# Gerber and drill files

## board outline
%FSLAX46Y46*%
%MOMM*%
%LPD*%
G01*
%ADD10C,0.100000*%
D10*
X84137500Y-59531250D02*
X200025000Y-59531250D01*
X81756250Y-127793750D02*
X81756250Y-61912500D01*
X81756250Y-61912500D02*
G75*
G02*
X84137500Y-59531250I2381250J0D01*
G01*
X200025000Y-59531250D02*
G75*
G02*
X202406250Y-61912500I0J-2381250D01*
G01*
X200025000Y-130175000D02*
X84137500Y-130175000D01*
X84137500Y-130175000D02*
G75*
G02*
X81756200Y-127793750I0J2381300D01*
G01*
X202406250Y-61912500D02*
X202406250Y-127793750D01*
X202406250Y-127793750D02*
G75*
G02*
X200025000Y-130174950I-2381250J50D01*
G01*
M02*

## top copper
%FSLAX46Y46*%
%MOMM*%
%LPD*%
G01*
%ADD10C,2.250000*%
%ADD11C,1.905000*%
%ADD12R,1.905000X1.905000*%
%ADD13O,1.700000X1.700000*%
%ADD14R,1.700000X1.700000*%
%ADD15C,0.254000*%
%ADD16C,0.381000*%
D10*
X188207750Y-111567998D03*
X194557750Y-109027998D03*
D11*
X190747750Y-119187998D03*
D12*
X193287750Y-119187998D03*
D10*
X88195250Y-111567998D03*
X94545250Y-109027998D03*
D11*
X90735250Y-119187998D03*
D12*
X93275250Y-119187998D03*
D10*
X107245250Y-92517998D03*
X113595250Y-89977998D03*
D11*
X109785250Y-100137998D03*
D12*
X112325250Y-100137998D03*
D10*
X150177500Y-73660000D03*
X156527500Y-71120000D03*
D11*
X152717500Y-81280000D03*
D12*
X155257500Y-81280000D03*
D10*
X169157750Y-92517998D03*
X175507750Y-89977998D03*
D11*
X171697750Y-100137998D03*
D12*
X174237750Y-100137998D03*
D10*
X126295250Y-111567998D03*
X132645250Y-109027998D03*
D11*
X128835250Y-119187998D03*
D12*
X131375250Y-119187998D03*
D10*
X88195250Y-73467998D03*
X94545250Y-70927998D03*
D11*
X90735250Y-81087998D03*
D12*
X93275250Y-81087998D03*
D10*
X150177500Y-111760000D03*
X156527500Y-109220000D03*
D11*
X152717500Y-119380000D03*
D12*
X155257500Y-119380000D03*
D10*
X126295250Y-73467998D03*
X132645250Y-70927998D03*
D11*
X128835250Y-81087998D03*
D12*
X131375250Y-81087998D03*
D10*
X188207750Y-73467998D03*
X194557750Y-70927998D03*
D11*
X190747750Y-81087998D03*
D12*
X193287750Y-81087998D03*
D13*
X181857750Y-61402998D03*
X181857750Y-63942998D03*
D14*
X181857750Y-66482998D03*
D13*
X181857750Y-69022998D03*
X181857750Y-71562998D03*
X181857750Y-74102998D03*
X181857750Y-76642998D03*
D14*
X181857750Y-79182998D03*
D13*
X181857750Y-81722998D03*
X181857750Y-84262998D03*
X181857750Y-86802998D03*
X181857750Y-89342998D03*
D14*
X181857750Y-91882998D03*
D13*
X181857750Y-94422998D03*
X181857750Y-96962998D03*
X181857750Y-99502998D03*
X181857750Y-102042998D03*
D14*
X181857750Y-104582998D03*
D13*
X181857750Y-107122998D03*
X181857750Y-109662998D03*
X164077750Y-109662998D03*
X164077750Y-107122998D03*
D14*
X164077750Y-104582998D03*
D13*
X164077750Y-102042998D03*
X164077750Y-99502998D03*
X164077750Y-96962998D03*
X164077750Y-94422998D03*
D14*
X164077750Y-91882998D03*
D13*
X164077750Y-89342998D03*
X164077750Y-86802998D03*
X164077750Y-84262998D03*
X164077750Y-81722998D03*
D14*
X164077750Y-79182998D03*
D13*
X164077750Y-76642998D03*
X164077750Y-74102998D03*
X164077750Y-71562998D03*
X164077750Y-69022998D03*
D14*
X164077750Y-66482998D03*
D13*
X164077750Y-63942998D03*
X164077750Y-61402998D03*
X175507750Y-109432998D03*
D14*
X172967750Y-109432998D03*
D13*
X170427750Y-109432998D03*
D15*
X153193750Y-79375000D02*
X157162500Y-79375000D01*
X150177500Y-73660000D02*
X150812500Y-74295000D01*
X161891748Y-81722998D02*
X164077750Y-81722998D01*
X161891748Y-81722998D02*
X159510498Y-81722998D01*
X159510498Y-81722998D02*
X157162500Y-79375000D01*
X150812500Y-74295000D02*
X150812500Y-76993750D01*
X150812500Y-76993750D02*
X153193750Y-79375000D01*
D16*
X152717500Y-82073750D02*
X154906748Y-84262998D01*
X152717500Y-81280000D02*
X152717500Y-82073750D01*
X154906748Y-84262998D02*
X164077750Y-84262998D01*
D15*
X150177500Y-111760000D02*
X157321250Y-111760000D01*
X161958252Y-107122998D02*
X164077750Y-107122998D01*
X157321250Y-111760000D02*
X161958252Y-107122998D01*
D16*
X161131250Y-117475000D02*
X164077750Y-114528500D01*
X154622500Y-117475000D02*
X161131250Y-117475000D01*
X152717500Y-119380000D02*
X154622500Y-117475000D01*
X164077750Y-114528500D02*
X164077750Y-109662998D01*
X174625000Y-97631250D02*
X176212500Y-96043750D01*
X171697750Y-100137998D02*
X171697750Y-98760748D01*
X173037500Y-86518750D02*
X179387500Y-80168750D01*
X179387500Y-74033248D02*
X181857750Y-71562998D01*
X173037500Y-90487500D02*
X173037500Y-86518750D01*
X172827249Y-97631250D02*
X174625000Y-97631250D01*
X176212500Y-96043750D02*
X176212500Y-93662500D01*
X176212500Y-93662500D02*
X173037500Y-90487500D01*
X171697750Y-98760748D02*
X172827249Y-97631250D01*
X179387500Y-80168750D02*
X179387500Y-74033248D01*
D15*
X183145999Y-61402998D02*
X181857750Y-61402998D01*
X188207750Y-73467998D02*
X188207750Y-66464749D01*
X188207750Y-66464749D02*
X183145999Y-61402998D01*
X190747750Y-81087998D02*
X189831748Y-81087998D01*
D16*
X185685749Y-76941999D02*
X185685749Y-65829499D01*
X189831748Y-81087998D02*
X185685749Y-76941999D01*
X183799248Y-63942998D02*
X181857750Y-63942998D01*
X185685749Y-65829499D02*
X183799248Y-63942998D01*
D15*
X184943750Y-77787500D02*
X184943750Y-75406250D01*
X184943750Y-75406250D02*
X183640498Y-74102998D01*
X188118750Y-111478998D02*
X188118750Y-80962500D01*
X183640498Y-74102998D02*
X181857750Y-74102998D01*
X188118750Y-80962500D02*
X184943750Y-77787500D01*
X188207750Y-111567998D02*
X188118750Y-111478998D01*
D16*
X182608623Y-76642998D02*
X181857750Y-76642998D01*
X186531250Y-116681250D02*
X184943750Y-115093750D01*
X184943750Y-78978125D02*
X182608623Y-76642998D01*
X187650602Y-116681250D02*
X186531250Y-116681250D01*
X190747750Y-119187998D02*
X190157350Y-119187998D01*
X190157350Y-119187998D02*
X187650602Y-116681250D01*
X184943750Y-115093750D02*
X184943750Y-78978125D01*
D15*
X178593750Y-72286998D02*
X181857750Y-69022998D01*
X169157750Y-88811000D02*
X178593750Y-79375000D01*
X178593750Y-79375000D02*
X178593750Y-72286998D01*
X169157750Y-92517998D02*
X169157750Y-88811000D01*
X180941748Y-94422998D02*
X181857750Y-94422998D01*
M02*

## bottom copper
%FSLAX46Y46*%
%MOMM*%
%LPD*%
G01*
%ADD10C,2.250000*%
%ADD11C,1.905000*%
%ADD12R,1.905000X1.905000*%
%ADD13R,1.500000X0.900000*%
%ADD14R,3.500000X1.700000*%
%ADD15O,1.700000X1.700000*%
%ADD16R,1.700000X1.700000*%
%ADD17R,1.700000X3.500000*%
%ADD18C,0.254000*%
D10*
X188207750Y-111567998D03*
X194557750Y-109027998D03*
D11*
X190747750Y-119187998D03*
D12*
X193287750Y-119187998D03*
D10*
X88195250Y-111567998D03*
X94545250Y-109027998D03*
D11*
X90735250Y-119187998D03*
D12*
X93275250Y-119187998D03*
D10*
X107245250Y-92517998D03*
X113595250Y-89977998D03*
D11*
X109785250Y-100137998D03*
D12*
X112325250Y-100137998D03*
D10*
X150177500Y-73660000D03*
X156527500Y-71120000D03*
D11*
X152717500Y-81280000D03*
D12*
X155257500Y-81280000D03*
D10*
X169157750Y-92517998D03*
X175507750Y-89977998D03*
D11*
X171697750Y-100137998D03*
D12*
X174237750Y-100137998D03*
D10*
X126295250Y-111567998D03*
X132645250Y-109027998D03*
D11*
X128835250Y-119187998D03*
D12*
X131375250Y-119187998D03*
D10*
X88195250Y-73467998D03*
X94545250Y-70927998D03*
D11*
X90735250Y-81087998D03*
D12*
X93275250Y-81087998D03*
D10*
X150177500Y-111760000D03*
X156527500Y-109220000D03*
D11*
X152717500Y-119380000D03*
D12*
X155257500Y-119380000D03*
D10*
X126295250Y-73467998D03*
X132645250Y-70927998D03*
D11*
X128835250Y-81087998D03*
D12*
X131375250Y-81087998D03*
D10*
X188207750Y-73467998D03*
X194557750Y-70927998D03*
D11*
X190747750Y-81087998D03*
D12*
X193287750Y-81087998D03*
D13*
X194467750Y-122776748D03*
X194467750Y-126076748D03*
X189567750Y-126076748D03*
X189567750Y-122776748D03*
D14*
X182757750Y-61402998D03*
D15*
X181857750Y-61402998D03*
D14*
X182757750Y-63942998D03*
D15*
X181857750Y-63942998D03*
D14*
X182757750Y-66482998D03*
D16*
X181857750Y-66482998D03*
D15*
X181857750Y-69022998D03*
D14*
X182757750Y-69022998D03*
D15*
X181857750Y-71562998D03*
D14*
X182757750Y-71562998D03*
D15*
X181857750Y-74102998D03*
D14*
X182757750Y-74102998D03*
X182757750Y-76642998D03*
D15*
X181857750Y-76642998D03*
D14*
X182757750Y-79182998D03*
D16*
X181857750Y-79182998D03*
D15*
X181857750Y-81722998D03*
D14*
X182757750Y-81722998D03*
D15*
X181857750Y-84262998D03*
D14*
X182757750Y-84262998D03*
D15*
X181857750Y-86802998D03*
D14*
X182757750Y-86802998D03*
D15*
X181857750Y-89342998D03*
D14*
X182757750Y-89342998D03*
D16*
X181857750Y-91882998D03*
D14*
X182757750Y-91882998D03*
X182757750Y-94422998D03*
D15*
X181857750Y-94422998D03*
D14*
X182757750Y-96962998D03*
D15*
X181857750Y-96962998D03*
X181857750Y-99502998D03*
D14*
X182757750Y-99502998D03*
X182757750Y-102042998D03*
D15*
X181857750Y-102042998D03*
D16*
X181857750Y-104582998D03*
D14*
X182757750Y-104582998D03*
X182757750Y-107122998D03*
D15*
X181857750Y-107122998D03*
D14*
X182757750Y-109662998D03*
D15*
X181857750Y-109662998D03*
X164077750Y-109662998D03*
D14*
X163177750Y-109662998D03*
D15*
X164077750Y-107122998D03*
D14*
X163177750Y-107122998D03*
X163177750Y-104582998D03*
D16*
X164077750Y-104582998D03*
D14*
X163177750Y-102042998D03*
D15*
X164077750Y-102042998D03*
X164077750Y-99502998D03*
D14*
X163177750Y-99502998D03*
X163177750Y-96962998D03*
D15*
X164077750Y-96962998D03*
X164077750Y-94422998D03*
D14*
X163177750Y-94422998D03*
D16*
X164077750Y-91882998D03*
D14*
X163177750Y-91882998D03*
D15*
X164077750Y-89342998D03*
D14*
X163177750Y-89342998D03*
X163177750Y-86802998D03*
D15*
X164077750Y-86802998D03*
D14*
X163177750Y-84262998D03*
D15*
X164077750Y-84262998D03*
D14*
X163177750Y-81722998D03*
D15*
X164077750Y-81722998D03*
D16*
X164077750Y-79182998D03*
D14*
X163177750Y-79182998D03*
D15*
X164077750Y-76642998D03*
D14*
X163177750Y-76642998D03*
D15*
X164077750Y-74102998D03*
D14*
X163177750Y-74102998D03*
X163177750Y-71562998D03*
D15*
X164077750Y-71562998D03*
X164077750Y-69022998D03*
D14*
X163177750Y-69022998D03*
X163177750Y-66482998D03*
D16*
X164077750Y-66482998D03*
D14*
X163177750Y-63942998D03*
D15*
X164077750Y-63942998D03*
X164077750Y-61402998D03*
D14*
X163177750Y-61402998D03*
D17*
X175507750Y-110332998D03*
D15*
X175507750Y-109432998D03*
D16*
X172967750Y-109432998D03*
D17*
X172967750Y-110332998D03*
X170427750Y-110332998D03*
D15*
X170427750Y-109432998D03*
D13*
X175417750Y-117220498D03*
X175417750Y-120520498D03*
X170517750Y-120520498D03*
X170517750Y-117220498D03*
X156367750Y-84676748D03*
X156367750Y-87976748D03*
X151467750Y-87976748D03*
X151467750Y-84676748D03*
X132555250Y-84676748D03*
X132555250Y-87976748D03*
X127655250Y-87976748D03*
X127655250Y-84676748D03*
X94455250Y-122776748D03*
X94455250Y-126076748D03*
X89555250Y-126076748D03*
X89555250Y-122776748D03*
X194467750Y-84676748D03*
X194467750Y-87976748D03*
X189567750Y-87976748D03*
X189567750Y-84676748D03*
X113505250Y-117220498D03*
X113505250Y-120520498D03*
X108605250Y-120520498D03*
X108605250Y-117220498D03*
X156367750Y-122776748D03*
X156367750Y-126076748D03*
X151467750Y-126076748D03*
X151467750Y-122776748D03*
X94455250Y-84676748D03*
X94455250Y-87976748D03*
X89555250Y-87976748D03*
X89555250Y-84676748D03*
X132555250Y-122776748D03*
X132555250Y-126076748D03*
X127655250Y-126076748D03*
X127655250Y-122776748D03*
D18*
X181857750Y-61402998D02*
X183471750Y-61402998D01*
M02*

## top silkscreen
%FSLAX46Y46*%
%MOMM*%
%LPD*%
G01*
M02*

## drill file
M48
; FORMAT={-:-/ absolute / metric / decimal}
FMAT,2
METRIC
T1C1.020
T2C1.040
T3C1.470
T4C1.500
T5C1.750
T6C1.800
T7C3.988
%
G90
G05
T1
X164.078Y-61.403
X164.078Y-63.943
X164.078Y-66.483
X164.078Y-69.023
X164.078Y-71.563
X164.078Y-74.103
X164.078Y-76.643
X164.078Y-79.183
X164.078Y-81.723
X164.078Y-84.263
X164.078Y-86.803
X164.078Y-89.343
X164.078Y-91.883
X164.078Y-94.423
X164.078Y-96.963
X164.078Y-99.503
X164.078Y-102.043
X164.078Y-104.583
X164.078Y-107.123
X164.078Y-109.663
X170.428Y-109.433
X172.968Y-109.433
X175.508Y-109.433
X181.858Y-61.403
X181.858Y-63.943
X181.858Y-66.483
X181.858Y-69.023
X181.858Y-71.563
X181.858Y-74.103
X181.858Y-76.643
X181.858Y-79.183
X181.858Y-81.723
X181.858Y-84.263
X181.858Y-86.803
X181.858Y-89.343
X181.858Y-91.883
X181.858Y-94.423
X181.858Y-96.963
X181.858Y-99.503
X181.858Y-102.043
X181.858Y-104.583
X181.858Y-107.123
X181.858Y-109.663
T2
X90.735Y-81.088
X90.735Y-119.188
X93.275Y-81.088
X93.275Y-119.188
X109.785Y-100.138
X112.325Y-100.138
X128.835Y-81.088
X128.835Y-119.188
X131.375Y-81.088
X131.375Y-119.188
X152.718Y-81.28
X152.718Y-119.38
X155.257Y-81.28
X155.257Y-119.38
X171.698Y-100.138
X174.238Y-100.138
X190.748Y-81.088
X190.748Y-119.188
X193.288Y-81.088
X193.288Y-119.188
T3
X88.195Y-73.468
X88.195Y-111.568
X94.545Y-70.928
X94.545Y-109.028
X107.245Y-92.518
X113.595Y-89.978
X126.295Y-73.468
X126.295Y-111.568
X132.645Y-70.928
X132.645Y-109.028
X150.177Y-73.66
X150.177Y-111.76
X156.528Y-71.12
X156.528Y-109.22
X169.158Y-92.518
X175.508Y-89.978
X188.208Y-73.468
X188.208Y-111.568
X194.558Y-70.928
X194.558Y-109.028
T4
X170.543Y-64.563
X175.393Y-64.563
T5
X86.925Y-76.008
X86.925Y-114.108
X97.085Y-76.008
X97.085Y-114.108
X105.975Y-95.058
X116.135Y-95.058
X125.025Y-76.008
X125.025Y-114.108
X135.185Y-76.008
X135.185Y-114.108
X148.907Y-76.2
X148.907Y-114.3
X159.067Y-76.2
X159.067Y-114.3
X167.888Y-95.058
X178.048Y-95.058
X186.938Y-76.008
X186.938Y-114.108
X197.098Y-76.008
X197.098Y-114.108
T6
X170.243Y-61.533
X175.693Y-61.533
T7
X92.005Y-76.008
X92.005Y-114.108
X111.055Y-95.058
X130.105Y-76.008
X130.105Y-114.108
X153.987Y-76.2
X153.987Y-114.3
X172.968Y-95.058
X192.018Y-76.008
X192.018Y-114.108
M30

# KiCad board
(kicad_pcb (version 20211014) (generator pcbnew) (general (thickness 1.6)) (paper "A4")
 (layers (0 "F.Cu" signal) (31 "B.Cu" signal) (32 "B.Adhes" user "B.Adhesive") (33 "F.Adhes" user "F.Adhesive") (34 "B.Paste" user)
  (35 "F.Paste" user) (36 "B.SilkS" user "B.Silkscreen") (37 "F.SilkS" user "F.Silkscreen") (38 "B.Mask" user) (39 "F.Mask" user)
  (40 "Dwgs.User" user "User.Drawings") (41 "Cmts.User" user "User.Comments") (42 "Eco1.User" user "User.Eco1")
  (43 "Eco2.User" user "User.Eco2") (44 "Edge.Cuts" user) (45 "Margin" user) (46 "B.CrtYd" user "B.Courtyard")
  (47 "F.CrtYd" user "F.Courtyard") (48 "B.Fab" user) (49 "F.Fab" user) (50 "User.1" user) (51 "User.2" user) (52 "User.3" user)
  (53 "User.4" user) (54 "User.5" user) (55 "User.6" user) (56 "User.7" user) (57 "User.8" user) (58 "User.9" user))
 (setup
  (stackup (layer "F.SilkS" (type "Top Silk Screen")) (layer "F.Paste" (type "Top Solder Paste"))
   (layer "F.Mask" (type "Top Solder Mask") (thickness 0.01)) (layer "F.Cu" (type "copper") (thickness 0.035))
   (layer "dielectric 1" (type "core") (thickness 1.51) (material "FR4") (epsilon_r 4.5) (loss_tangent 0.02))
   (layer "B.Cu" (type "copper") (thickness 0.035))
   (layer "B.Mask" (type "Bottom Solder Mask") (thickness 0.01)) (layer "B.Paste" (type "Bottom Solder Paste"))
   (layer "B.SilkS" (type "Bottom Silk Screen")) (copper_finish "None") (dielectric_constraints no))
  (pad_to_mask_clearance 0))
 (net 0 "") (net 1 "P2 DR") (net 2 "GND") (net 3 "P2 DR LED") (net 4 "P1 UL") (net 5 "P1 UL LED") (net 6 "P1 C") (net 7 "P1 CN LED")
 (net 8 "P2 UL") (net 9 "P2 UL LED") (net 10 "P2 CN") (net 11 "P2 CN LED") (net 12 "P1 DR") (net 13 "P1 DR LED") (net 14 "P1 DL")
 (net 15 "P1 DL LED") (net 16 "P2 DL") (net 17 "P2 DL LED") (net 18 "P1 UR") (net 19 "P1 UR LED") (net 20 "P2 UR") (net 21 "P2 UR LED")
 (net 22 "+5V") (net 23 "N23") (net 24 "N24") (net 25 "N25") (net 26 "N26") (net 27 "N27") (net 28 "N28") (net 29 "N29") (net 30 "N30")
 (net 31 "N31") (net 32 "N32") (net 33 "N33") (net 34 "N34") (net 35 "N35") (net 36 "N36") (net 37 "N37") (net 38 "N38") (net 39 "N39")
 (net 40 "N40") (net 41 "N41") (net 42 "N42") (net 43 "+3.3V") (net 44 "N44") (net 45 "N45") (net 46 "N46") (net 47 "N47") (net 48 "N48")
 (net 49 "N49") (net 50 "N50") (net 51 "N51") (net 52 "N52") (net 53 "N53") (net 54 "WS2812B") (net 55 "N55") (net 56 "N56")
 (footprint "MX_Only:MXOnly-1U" (layer "F.Cu") (at 192.01775 114.107998)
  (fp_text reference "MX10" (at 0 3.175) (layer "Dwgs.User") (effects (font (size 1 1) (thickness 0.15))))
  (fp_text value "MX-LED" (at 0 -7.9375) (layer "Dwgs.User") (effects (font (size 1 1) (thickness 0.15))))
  (pad "" np_thru_hole circle locked (at 0 0) (size 3.9878 3.9878) (drill 3.9878) (layers *.Cu *.Mask))
  (pad "" np_thru_hole circle locked (at 5.08 0 48.0996) (size 1.75 1.75) (drill 1.75) (layers *.Cu *.Mask))
  (pad "" np_thru_hole circle locked (at -5.08 0 48.0996) (size 1.75 1.75) (drill 1.75) (layers *.Cu *.Mask))
  (pad "1" thru_hole circle locked (at -3.81 -2.54) (size 2.25 2.25) (drill 1.47) (layers *.Cu "B.Mask") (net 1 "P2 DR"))
  (pad "2" thru_hole circle locked (at 2.54 -5.08) (size 2.25 2.25) (drill 1.47) (layers *.Cu "B.Mask") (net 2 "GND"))
  (pad "3" thru_hole circle locked (at -1.27 5.08) (size 1.905 1.905) (drill 1.04) (layers *.Cu "B.Mask") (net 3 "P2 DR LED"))
  (pad "4" thru_hole rect locked (at 1.27 5.08) (size 1.905 1.905) (drill 1.04) (layers *.Cu "B.Mask") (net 2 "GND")))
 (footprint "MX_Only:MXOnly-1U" (layer "F.Cu") (at 92.00525 114.107998)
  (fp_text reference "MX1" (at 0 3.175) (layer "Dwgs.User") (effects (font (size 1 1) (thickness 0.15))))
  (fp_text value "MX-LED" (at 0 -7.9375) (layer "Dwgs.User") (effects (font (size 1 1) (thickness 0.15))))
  (pad "" np_thru_hole circle locked (at -5.08 0 48.0996) (size 1.75 1.75) (drill 1.75) (layers *.Cu *.Mask))
  (pad "" np_thru_hole circle locked (at 5.08 0 48.0996) (size 1.75 1.75) (drill 1.75) (layers *.Cu *.Mask))
  (pad "" np_thru_hole circle locked (at 0 0) (size 3.9878 3.9878) (drill 3.9878) (layers *.Cu *.Mask))
  (pad "1" thru_hole circle locked (at -3.81 -2.54) (size 2.25 2.25) (drill 1.47) (layers *.Cu "B.Mask") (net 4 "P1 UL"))
  (pad "2" thru_hole circle locked (at 2.54 -5.08) (size 2.25 2.25) (drill 1.47) (layers *.Cu "B.Mask") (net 2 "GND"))
  (pad "3" thru_hole circle locked (at -1.27 5.08) (size 1.905 1.905) (drill 1.04) (layers *.Cu "B.Mask") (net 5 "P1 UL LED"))
  (pad "4" thru_hole rect locked (at 1.27 5.08) (size 1.905 1.905) (drill 1.04) (layers *.Cu "B.Mask") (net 2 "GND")))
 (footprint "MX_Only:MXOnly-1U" (layer "F.Cu") (at 111.05525 95.057998)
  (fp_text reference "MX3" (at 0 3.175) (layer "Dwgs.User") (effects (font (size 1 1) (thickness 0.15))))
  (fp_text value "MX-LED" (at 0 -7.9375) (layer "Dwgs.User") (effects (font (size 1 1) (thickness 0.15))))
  (pad "" np_thru_hole circle locked (at -5.08 0 48.0996) (size 1.75 1.75) (drill 1.75) (layers *.Cu *.Mask))
  (pad "" np_thru_hole circle locked (at 5.08 0 48.0996) (size 1.75 1.75) (drill 1.75) (layers *.Cu *.Mask))
  (pad "" np_thru_hole circle locked (at 0 0) (size 3.9878 3.9878) (drill 3.9878) (layers *.Cu *.Mask))
  (pad "1" thru_hole circle locked (at -3.81 -2.54) (size 2.25 2.25) (drill 1.47) (layers *.Cu "B.Mask") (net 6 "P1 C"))
  (pad "2" thru_hole circle locked (at 2.54 -5.08) (size 2.25 2.25) (drill 1.47) (layers *.Cu "B.Mask") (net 2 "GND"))
  (pad "3" thru_hole circle locked (at -1.27 5.08) (size 1.905 1.905) (drill 1.04) (layers *.Cu "B.Mask") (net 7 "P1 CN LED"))
  (pad "4" thru_hole rect locked (at 1.27 5.08) (size 1.905 1.905) (drill 1.04) (layers *.Cu "B.Mask") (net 2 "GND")))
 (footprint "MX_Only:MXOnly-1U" (layer "F.Cu") (at 153.9875 76.2)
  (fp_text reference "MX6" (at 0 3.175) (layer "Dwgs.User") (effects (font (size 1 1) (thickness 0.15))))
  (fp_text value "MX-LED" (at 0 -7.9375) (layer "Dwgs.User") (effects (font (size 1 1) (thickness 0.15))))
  (pad "" np_thru_hole circle locked (at -5.08 0 48.0996) (size 1.75 1.75) (drill 1.75) (layers *.Cu *.Mask))
  (pad "" np_thru_hole circle locked (at 0 0) (size 3.9878 3.9878) (drill 3.9878) (layers *.Cu *.Mask))
  (pad "" np_thru_hole circle locked (at 5.08 0 48.0996) (size 1.75 1.75) (drill 1.75) (layers *.Cu *.Mask))
  (pad "1" thru_hole circle locked (at -3.81 -2.54) (size 2.25 2.25) (drill 1.47) (layers *.Cu "B.Mask") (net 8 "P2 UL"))
  (pad "2" thru_hole circle locked (at 2.54 -5.08) (size 2.25 2.25) (drill 1.47) (layers *.Cu "B.Mask") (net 2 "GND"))
  (pad "3" thru_hole circle locked (at -1.27 5.08) (size 1.905 1.905) (drill 1.04) (layers *.Cu "B.Mask") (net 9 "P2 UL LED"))
  (pad "4" thru_hole rect locked (at 1.27 5.08) (size 1.905 1.905) (drill 1.04) (layers *.Cu "B.Mask") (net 2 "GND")))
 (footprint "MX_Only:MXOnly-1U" (layer "F.Cu") (at 172.96775 95.057998)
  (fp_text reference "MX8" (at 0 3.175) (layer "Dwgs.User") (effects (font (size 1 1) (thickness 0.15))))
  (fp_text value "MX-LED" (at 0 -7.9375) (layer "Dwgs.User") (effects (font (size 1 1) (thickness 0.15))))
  (pad "" np_thru_hole circle locked (at 5.08 0 48.0996) (size 1.75 1.75) (drill 1.75) (layers *.Cu *.Mask))
  (pad "" np_thru_hole circle locked (at -5.08 0 48.0996) (size 1.75 1.75) (drill 1.75) (layers *.Cu *.Mask))
  (pad "" np_thru_hole circle locked (at 0 0) (size 3.9878 3.9878) (drill 3.9878) (layers *.Cu *.Mask))
  (pad "1" thru_hole circle locked (at -3.81 -2.54) (size 2.25 2.25) (drill 1.47) (layers *.Cu "B.Mask") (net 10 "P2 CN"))
  (pad "2" thru_hole circle locked (at 2.54 -5.08) (size 2.25 2.25) (drill 1.47) (layers *.Cu "B.Mask") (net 2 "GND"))
  (pad "3" thru_hole circle locked (at -1.27 5.08) (size 1.905 1.905) (drill 1.04) (layers *.Cu "B.Mask") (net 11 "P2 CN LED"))
  (pad "4" thru_hole rect locked (at 1.27 5.08) (size 1.905 1.905) (drill 1.04) (layers *.Cu "B.Mask") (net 2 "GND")))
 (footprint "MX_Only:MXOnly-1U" (layer "F.Cu") (at 130.10525 114.107998)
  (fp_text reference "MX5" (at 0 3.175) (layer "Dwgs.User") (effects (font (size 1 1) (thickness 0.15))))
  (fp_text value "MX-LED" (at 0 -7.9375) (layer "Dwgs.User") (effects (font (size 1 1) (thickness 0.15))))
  (pad "" np_thru_hole circle locked (at 5.08 0 48.0996) (size 1.75 1.75) (drill 1.75) (layers *.Cu *.Mask))
  (pad "" np_thru_hole circle locked (at -5.08 0 48.0996) (size 1.75 1.75) (drill 1.75) (layers *.Cu *.Mask))
  (pad "" np_thru_hole circle locked (at 0 0) (size 3.9878 3.9878) (drill 3.9878) (layers *.Cu *.Mask))
  (pad "1" thru_hole circle locked (at -3.81 -2.54) (size 2.25 2.25) (drill 1.47) (layers *.Cu "B.Mask") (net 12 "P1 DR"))
  (pad "2" thru_hole circle locked (at 2.54 -5.08) (size 2.25 2.25) (drill 1.47) (layers *.Cu "B.Mask") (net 2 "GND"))
  (pad "3" thru_hole circle locked (at -1.27 5.08) (size 1.905 1.905) (drill 1.04) (layers *.Cu "B.Mask") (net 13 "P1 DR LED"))
  (pad "4" thru_hole rect locked (at 1.27 5.08) (size 1.905 1.905) (drill 1.04) (layers *.Cu "B.Mask") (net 2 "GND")))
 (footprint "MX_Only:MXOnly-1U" (layer "F.Cu") (at 92.00525 76.007998)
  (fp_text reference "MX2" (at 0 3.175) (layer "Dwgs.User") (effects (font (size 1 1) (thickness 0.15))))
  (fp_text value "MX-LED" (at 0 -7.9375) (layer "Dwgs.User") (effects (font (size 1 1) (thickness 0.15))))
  (pad "" np_thru_hole circle locked (at 0 0) (size 3.9878 3.9878) (drill 3.9878) (layers *.Cu *.Mask))
  (pad "" np_thru_hole circle locked (at -5.08 0 48.0996) (size 1.75 1.75) (drill 1.75) (layers *.Cu *.Mask))
  (pad "" np_thru_hole circle locked (at 5.08 0 48.0996) (size 1.75 1.75) (drill 1.75) (layers *.Cu *.Mask))
  (pad "1" thru_hole circle locked (at -3.81 -2.54) (size 2.25 2.25) (drill 1.47) (layers *.Cu "B.Mask") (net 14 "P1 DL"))
  (pad "2" thru_hole circle locked (at 2.54 -5.08) (size 2.25 2.25) (drill 1.47) (layers *.Cu "B.Mask") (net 2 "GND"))
  (pad "3" thru_hole circle locked (at -1.27 5.08) (size 1.905 1.905) (drill 1.04) (layers *.Cu "B.Mask") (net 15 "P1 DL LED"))
  (pad "4" thru_hole rect locked (at 1.27 5.08) (size 1.905 1.905) (drill 1.04) (layers *.Cu "B.Mask") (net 2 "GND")))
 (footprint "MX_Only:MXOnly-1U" (layer "F.Cu") (at 153.9875 114.3)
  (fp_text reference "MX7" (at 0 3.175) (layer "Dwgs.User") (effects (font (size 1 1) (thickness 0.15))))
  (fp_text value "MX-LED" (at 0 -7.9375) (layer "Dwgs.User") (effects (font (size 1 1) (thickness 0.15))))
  (pad "" np_thru_hole circle locked (at -5.08 0 48.0996) (size 1.75 1.75) (drill 1.75) (layers *.Cu *.Mask))
  (pad "" np_thru_hole circle locked (at 5.08 0 48.0996) (size 1.75 1.75) (drill 1.75) (layers *.Cu *.Mask))
  (pad "" np_thru_hole circle locked (at 0 0) (size 3.9878 3.9878) (drill 3.9878) (layers *.Cu *.Mask))
  (pad "1" thru_hole circle locked (at -3.81 -2.54) (size 2.25 2.25) (drill 1.47) (layers *.Cu "B.Mask") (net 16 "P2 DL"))
  (pad "2" thru_hole circle locked (at 2.54 -5.08) (size 2.25 2.25) (drill 1.47) (layers *.Cu "B.Mask") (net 2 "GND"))
  (pad "3" thru_hole circle locked (at -1.27 5.08) (size 1.905 1.905) (drill 1.04) (layers *.Cu "B.Mask") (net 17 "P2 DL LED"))
  (pad "4" thru_hole rect locked (at 1.27 5.08) (size 1.905 1.905) (drill 1.04) (layers *.Cu "B.Mask") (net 2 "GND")))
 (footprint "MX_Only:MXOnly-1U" (layer "F.Cu") (at 130.10525 76.007998)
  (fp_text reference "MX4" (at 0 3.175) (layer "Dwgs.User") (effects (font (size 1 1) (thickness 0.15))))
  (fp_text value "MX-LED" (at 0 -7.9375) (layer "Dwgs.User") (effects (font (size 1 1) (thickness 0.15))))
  (pad "" np_thru_hole circle locked (at -5.08 0 48.0996) (size 1.75 1.75) (drill 1.75) (layers *.Cu *.Mask))
  (pad "" np_thru_hole circle locked (at 5.08 0 48.0996) (size 1.75 1.75) (drill 1.75) (layers *.Cu *.Mask))
  (pad "" np_thru_hole circle locked (at 0 0) (size 3.9878 3.9878) (drill 3.9878) (layers *.Cu *.Mask))
  (pad "1" thru_hole circle locked (at -3.81 -2.54) (size 2.25 2.25) (drill 1.47) (layers *.Cu "B.Mask") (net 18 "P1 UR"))
  (pad "2" thru_hole circle locked (at 2.54 -5.08) (size 2.25 2.25) (drill 1.47) (layers *.Cu "B.Mask") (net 2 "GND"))
  (pad "3" thru_hole circle locked (at -1.27 5.08) (size 1.905 1.905) (drill 1.04) (layers *.Cu "B.Mask") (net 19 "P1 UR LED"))
  (pad "4" thru_hole rect locked (at 1.27 5.08) (size 1.905 1.905) (drill 1.04) (layers *.Cu "B.Mask") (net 2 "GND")))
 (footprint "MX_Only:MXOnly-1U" (layer "F.Cu") (at 192.01775 76.007998)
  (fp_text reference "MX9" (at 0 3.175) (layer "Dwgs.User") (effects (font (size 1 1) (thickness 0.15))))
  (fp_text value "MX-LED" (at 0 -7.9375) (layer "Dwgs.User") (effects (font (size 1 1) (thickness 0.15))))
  (pad "" np_thru_hole circle locked (at -5.08 0 48.0996) (size 1.75 1.75) (drill 1.75) (layers *.Cu *.Mask))
  (pad "" np_thru_hole circle locked (at 5.08 0 48.0996) (size 1.75 1.75) (drill 1.75) (layers *.Cu *.Mask))
  (pad "" np_thru_hole circle locked (at 0 0) (size 3.9878 3.9878) (drill 3.9878) (layers *.Cu *.Mask))
  (pad "1" thru_hole circle locked (at -3.81 -2.54) (size 2.25 2.25) (drill 1.47) (layers *.Cu "B.Mask") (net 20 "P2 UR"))
  (pad "2" thru_hole circle locked (at 2.54 -5.08) (size 2.25 2.25) (drill 1.47) (layers *.Cu "B.Mask") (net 2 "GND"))
  (pad "3" thru_hole circle locked (at -1.27 5.08) (size 1.905 1.905) (drill 1.04) (layers *.Cu "B.Mask") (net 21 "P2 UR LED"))
  (pad "4" thru_hole rect locked (at 1.27 5.08) (size 1.905 1.905) (drill 1.04) (layers *.Cu "B.Mask") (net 2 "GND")))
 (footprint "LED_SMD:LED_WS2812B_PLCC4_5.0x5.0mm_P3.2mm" (layer "B.Cu") (at 192.01775 124.426748 180)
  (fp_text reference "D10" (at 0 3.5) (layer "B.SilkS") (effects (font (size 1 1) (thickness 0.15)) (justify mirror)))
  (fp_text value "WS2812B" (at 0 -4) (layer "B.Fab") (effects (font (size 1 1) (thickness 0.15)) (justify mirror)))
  (pad "1" smd rect (at -2.45 1.65 180) (size 1.5 0.9) (layers "B.Cu" "B.Paste" "B.Mask") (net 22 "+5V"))
  (pad "2" smd rect (at -2.45 -1.65 180) (size 1.5 0.9) (layers "B.Cu" "B.Paste" "B.Mask") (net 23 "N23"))
  (pad "3" smd rect (at 2.45 -1.65 180) (size 1.5 0.9) (layers "B.Cu" "B.Paste" "B.Mask") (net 2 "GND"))
  (pad "4" smd rect (at 2.45 1.65 180) (size 1.5 0.9) (layers "B.Cu" "B.Paste" "B.Mask") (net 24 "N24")))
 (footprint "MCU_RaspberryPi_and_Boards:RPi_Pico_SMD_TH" (layer "B.Cu") (at 172.96775 85.532998 180)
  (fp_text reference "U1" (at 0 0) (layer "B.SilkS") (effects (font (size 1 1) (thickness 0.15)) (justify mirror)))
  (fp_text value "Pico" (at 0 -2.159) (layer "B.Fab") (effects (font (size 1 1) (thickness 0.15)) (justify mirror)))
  (pad "" np_thru_hole oval (at 2.725 24 180) (size 1.8 1.8) (drill 1.8) (layers *.Cu *.Mask))
  (pad "" np_thru_hole oval (at -2.425 20.97 180) (size 1.5 1.5) (drill 1.5) (layers *.Cu *.Mask))
  (pad "" np_thru_hole oval (at 2.425 20.97 180) (size 1.5 1.5) (drill 1.5) (layers *.Cu *.Mask))
  (pad "" np_thru_hole oval (at -2.725 24 180) (size 1.8 1.8) (drill 1.8) (layers *.Cu *.Mask))
  (pad "1" smd rect (at -8.89 24.13 180) (size 3.5 1.7) (drill (offset -0.9 0)) (layers "B.Cu" "B.Mask") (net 20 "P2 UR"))
  (pad "1" thru_hole oval (at -8.89 24.13 180) (size 1.7 1.7) (drill 1.02) (layers *.Cu *.Mask) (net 20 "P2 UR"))
  (pad "2" smd rect (at -8.89 21.59 180) (size 3.5 1.7) (drill (offset -0.9 0)) (layers "B.Cu" "B.Mask") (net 21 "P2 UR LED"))
  (pad "2" thru_hole oval (at -8.89 21.59 180) (size 1.7 1.7) (drill 1.02) (layers *.Cu *.Mask) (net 21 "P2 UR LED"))
  (pad "3" smd rect (at -8.89 19.05 180) (size 3.5 1.7) (drill (offset -0.9 0)) (layers "B.Cu" "B.Mask") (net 2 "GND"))
  (pad "3" thru_hole rect (at -8.89 19.05 180) (size 1.7 1.7) (drill 1.02) (layers *.Cu *.Mask) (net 2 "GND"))
  (pad "4" thru_hole oval (at -8.89 16.51 180) (size 1.7 1.7) (drill 1.02) (layers *.Cu *.Mask) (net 10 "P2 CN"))
  (pad "4" smd rect (at -8.89 16.51 180) (size 3.5 1.7) (drill (offset -0.9 0)) (layers "B.Cu" "B.Mask") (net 10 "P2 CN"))
  (pad "5" thru_hole oval (at -8.89 13.97 180) (size 1.7 1.7) (drill 1.02) (layers *.Cu *.Mask) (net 11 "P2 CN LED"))
  (pad "5" smd rect (at -8.89 13.97 180) (size 3.5 1.7) (drill (offset -0.9 0)) (layers "B.Cu" "B.Mask") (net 11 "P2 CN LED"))
  (pad "6" thru_hole oval (at -8.89 11.43 180) (size 1.7 1.7) (drill 1.02) (layers *.Cu *.Mask) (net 1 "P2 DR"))
  (pad "6" smd rect (at -8.89 11.43 180) (size 3.5 1.7) (drill (offset -0.9 0)) (layers "B.Cu" "B.Mask") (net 1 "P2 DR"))
  (pad "7" smd rect (at -8.89 8.89 180) (size 3.5 1.7) (drill (offset -0.9 0)) (layers "B.Cu" "B.Mask") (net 3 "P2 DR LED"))
  (pad "7" thru_hole oval (at -8.89 8.89 180) (size 1.7 1.7) (drill 1.02) (layers *.Cu *.Mask) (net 3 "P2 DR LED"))
  (pad "8" smd rect (at -8.89 6.35 180) (size 3.5 1.7) (drill (offset -0.9 0)) (layers "B.Cu" "B.Mask") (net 2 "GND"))
  (pad "8" thru_hole rect (at -8.89 6.35 180) (size 1.7 1.7) (drill 1.02) (layers *.Cu *.Mask) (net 2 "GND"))
  (pad "9" thru_hole oval (at -8.89 3.81 180) (size 1.7 1.7) (drill 1.02) (layers *.Cu *.Mask) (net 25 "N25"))
  (pad "9" smd rect (at -8.89 3.81 180) (size 3.5 1.7) (drill (offset -0.9 0)) (layers "B.Cu" "B.Mask") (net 25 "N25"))
  (pad "10" thru_hole oval (at -8.89 1.27 180) (size 1.7 1.7) (drill 1.02) (layers *.Cu *.Mask) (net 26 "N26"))
  (pad "10" smd rect (at -8.89 1.27 180) (size 3.5 1.7) (drill (offset -0.9 0)) (layers "B.Cu" "B.Mask") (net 26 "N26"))
  (pad "11" thru_hole oval (at -8.89 -1.27 180) (size 1.7 1.7) (drill 1.02) (layers *.Cu *.Mask) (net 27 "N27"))
  (pad "11" smd rect (at -8.89 -1.27 180) (size 3.5 1.7) (drill (offset -0.9 0)) (layers "B.Cu" "B.Mask") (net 27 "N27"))
  (pad "12" thru_hole oval (at -8.89 -3.81 180) (size 1.7 1.7) (drill 1.02) (layers *.Cu *.Mask) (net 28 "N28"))
  (pad "12" smd rect (at -8.89 -3.81 180) (size 3.5 1.7) (drill (offset -0.9 0)) (layers "B.Cu" "B.Mask") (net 28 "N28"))
  (pad "13" thru_hole rect (at -8.89 -6.35 180) (size 1.7 1.7) (drill 1.02) (layers *.Cu *.Mask) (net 2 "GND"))
  (pad "13" smd rect (at -8.89 -6.35 180) (size 3.5 1.7) (drill (offset -0.9 0)) (layers "B.Cu" "B.Mask") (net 2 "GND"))
  (pad "14" smd rect (at -8.89 -8.89 180) (size 3.5 1.7) (drill (offset -0.9 0)) (layers "B.Cu" "B.Mask") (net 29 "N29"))
  (pad "14" thru_hole oval (at -8.89 -8.89 180) (size 1.7 1.7) (drill 1.02) (layers *.Cu *.Mask) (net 29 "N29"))
  (pad "15" smd rect (at -8.89 -11.43 180) (size 3.5 1.7) (drill (offset -0.9 0)) (layers "B.Cu" "B.Mask") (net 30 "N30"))
  (pad "15" thru_hole oval (at -8.89 -11.43 180) (size 1.7 1.7) (drill 1.02) (layers *.Cu *.Mask) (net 30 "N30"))
  (pad "16" thru_hole oval (at -8.89 -13.97 180) (size 1.7 1.7) (drill 1.02) (layers *.Cu *.Mask) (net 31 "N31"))
  (pad "16" smd rect (at -8.89 -13.97 180) (size 3.5 1.7) (drill (offset -0.9 0)) (layers "B.Cu" "B.Mask") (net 31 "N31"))
  (pad "17" smd rect (at -8.89 -16.51 180) (size 3.5 1.7) (drill (offset -0.9 0)) (layers "B.Cu" "B.Mask") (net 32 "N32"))
  (pad "17" thru_hole oval (at -8.89 -16.51 180) (size 1.7 1.7) (drill 1.02) (layers *.Cu *.Mask) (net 32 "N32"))
  (pad "18" thru_hole rect (at -8.89 -19.05 180) (size 1.7 1.7) (drill 1.02) (layers *.Cu *.Mask) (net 2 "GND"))
  (pad "18" smd rect (at -8.89 -19.05 180) (size 3.5 1.7) (drill (offset -0.9 0)) (layers "B.Cu" "B.Mask") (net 2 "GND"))
  (pad "19" smd rect (at -8.89 -21.59 180) (size 3.5 1.7) (drill (offset -0.9 0)) (layers "B.Cu" "B.Mask") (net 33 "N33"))
  (pad "19" thru_hole oval (at -8.89 -21.59 180) (size 1.7 1.7) (drill 1.02) (layers *.Cu *.Mask) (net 33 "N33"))
  (pad "20" smd rect (at -8.89 -24.13 180) (size 3.5 1.7) (drill (offset -0.9 0)) (layers "B.Cu" "B.Mask") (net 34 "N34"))
  (pad "20" thru_hole oval (at -8.89 -24.13 180) (size 1.7 1.7) (drill 1.02) (layers *.Cu *.Mask) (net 34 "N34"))
  (pad "21" thru_hole oval (at 8.89 -24.13 180) (size 1.7 1.7) (drill 1.02) (layers *.Cu *.Mask) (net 17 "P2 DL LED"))
  (pad "21" smd rect (at 8.89 -24.13 180) (size 3.5 1.7) (drill (offset 0.9 0)) (layers "B.Cu" "B.Mask") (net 17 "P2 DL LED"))
  (pad "22" thru_hole oval (at 8.89 -21.59 180) (size 1.7 1.7) (drill 1.02) (layers *.Cu *.Mask) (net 16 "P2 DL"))
  (pad "22" smd rect (at 8.89 -21.59 180) (size 3.5 1.7) (drill (offset 0.9 0)) (layers "B.Cu" "B.Mask") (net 16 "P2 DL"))
  (pad "23" smd rect (at 8.89 -19.05 180) (size 3.5 1.7) (drill (offset 0.9 0)) (layers "B.Cu" "B.Mask") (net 2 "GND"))
  (pad "23" thru_hole rect (at 8.89 -19.05 180) (size 1.7 1.7) (drill 1.02) (layers *.Cu *.Mask) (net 2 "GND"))
  (pad "24" smd rect (at 8.89 -16.51 180) (size 3.5 1.7) (drill (offset 0.9 0)) (layers "B.Cu" "B.Mask") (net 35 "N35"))
  (pad "24" thru_hole oval (at 8.89 -16.51 180) (size 1.7 1.7) (drill 1.02) (layers *.Cu *.Mask) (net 35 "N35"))
  (pad "25" thru_hole oval (at 8.89 -13.97 180) (size 1.7 1.7) (drill 1.02) (layers *.Cu *.Mask) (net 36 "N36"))
  (pad "25" smd rect (at 8.89 -13.97 180) (size 3.5 1.7) (drill (offset 0.9 0)) (layers "B.Cu" "B.Mask") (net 36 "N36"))
  (pad "26" smd rect (at 8.89 -11.43 180) (size 3.5 1.7) (drill (offset 0.9 0)) (layers "B.Cu" "B.Mask") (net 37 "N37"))
  (pad "26" thru_hole oval (at 8.89 -11.43 180) (size 1.7 1.7) (drill 1.02) (layers *.Cu *.Mask) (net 37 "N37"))
  (pad "27" thru_hole oval (at 8.89 -8.89 180) (size 1.7 1.7) (drill 1.02) (layers *.Cu *.Mask) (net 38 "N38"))
  (pad "27" smd rect (at 8.89 -8.89 180) (size 3.5 1.7) (drill (offset 0.9 0)) (layers "B.Cu" "B.Mask") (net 38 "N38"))
  (pad "28" thru_hole rect (at 8.89 -6.35 180) (size 1.7 1.7) (drill 1.02) (layers *.Cu *.Mask) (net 2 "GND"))
  (pad "28" smd rect (at 8.89 -6.35 180) (size 3.5 1.7) (drill (offset 0.9 0)) (layers "B.Cu" "B.Mask") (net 2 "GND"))
  (pad "29" thru_hole oval (at 8.89 -3.81 180) (size 1.7 1.7) (drill 1.02) (layers *.Cu *.Mask) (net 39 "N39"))
  (pad "29" smd rect (at 8.89 -3.81 180) (size 3.5 1.7) (drill (offset 0.9 0)) (layers "B.Cu" "B.Mask") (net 39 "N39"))
  (pad "30" smd rect (at 8.89 -1.27 180) (size 3.5 1.7) (drill (offset 0.9 0)) (layers "B.Cu" "B.Mask") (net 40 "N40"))
  (pad "30" thru_hole oval (at 8.89 -1.27 180) (size 1.7 1.7) (drill 1.02) (layers *.Cu *.Mask) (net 40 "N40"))
  (pad "31" smd rect (at 8.89 1.27 180) (size 3.5 1.7) (drill (offset 0.9 0)) (layers "B.Cu" "B.Mask") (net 9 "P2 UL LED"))
  (pad "31" thru_hole oval (at 8.89 1.27 180) (size 1.7 1.7) (drill 1.02) (layers *.Cu *.Mask) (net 9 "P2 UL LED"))
  (pad "32" smd rect (at 8.89 3.81 180) (size 3.5 1.7) (drill (offset 0.9 0)) (layers "B.Cu" "B.Mask") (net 8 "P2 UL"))
  (pad "32" thru_hole oval (at 8.89 3.81 180) (size 1.7 1.7) (drill 1.02) (layers *.Cu *.Mask) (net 8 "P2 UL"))
  (pad "33" thru_hole rect (at 8.89 6.35 180) (size 1.7 1.7) (drill 1.02) (layers *.Cu *.Mask) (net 2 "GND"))
  (pad "33" smd rect (at 8.89 6.35 180) (size 3.5 1.7) (drill (offset 0.9 0)) (layers "B.Cu" "B.Mask") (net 2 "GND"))
  (pad "34" thru_hole oval (at 8.89 8.89 180) (size 1.7 1.7) (drill 1.02) (layers *.Cu *.Mask) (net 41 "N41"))
  (pad "34" smd rect (at 8.89 8.89 180) (size 3.5 1.7) (drill (offset 0.9 0)) (layers "B.Cu" "B.Mask") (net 41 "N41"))
  (pad "35" thru_hole oval (at 8.89 11.43 180) (size 1.7 1.7) (drill 1.02) (layers *.Cu *.Mask) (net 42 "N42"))
  (pad "35" smd rect (at 8.89 11.43 180) (size 3.5 1.7) (drill (offset 0.9 0)) (layers "B.Cu" "B.Mask") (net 42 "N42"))
  (pad "36" smd rect (at 8.89 13.97 180) (size 3.5 1.7) (drill (offset 0.9 0)) (layers "B.Cu" "B.Mask") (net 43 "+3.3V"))
  (pad "36" thru_hole oval (at 8.89 13.97 180) (size 1.7 1.7) (drill 1.02) (layers *.Cu *.Mask) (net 43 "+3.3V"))
  (pad "37" thru_hole oval (at 8.89 16.51 180) (size 1.7 1.7) (drill 1.02) (layers *.Cu *.Mask) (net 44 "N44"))
  (pad "37" smd rect (at 8.89 16.51 180) (size 3.5 1.7) (drill (offset 0.9 0)) (layers "B.Cu" "B.Mask") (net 44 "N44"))
  (pad "38" smd rect (at 8.89 19.05 180) (size 3.5 1.7) (drill (offset 0.9 0)) (layers "B.Cu" "B.Mask") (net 2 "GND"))
  (pad "38" thru_hole rect (at 8.89 19.05 180) (size 1.7 1.7) (drill 1.02) (layers *.Cu *.Mask) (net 2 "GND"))
  (pad "39" smd rect (at 8.89 21.59 180) (size 3.5 1.7) (drill (offset 0.9 0)) (layers "B.Cu" "B.Mask") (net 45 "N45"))
  (pad "39" thru_hole oval (at 8.89 21.59 180) (size 1.7 1.7) (drill 1.02) (layers *.Cu *.Mask) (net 45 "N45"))
  (pad "40" thru_hole oval (at 8.89 24.13 180) (size 1.7 1.7) (drill 1.02) (layers *.Cu *.Mask) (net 22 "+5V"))
  (pad "40" smd rect (at 8.89 24.13 180) (size 3.5 1.7) (drill (offset 0.9 0)) (layers "B.Cu" "B.Mask") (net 22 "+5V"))
  (pad "41" smd rect (at -2.54 -23.9 90) (size 3.5 1.7) (drill (offset -0.9 0)) (layers "B.Cu" "B.Mask") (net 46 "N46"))
  (pad "41" thru_hole oval (at -2.54 -23.9 180) (size 1.7 1.7) (drill 1.02) (layers *.Cu *.Mask) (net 46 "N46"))
  (pad "42" thru_hole rect (at 0 -23.9 180) (size 1.7 1.7) (drill 1.02) (layers *.Cu *.Mask) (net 2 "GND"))
  (pad "42" smd rect (at 0 -23.9 90) (size 3.5 1.7) (drill (offset -0.9 0)) (layers "B.Cu" "B.Mask") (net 2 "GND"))
  (pad "43" smd rect (at 2.54 -23.9 90) (size 3.5 1.7) (drill (offset -0.9 0)) (layers "B.Cu" "B.Mask") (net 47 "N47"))
  (pad "43" thru_hole oval (at 2.54 -23.9 180) (size 1.7 1.7) (drill 1.02) (layers *.Cu *.Mask) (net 47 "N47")))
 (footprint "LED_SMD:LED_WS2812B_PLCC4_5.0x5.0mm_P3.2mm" (layer "B.Cu") (at 172.96775 118.870498 180)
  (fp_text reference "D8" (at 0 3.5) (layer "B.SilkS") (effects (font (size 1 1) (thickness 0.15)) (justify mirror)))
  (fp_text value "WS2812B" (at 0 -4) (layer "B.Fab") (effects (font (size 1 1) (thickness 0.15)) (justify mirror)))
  (pad "1" smd rect (at -2.45 1.65 180) (size 1.5 0.9) (layers "B.Cu" "B.Paste" "B.Mask") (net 22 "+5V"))
  (pad "2" smd rect (at -2.45 -1.65 180) (size 1.5 0.9) (layers "B.Cu" "B.Paste" "B.Mask") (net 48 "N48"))
  (pad "3" smd rect (at 2.45 -1.65 180) (size 1.5 0.9) (layers "B.Cu" "B.Paste" "B.Mask") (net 2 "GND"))
  (pad "4" smd rect (at 2.45 1.65 180) (size 1.5 0.9) (layers "B.Cu" "B.Paste" "B.Mask") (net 23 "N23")))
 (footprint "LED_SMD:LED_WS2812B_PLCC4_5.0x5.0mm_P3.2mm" (layer "B.Cu") (at 153.91775 86.326748 180)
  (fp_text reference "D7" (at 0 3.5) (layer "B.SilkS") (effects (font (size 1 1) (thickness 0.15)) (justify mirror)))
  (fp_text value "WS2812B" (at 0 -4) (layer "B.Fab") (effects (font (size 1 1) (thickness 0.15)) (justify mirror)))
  (pad "1" smd rect (at -2.45 1.65 180) (size 1.5 0.9) (layers "B.Cu" "B.Paste" "B.Mask") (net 22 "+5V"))
  (pad "2" smd rect (at -2.45 -1.65 180) (size 1.5 0.9) (layers "B.Cu" "B.Paste" "B.Mask") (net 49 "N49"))
  (pad "3" smd rect (at 2.45 -1.65 180) (size 1.5 0.9) (layers "B.Cu" "B.Paste" "B.Mask") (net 2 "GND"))
  (pad "4" smd rect (at 2.45 1.65 180) (size 1.5 0.9) (layers "B.Cu" "B.Paste" "B.Mask") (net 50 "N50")))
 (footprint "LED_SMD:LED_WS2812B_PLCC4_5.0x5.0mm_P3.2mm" (layer "B.Cu") (at 130.10525 86.326748 180)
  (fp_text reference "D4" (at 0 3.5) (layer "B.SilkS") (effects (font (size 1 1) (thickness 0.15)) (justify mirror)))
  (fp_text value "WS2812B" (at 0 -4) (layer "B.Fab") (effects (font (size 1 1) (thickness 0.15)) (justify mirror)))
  (pad "1" smd rect (at -2.45 1.65 180) (size 1.5 0.9) (layers "B.Cu" "B.Paste" "B.Mask") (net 22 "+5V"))
  (pad "2" smd rect (at -2.45 -1.65 180) (size 1.5 0.9) (layers "B.Cu" "B.Paste" "B.Mask") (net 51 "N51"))
  (pad "3" smd rect (at 2.45 -1.65 180) (size 1.5 0.9) (layers "B.Cu" "B.Paste" "B.Mask") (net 2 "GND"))
  (pad "4" smd rect (at 2.45 1.65 180) (size 1.5 0.9) (layers "B.Cu" "B.Paste" "B.Mask") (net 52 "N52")))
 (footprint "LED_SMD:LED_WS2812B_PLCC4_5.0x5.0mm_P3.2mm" (layer "B.Cu") (at 92.00525 124.426748 180)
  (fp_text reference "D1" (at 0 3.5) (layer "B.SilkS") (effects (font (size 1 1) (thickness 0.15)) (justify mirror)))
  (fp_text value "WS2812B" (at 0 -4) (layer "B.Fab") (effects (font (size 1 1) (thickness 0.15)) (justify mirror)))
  (pad "1" smd rect (at -2.45 1.65 180) (size 1.5 0.9) (layers "B.Cu" "B.Paste" "B.Mask") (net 22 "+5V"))
  (pad "2" smd rect (at -2.45 -1.65 180) (size 1.5 0.9) (layers "B.Cu" "B.Paste" "B.Mask") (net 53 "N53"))
  (pad "3" smd rect (at 2.45 -1.65 180) (size 1.5 0.9) (layers "B.Cu" "B.Paste" "B.Mask") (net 2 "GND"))
  (pad "4" smd rect (at 2.45 1.65 180) (size 1.5 0.9) (layers "B.Cu" "B.Paste" "B.Mask") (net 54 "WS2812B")))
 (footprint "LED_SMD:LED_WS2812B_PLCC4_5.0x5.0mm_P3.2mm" (layer "B.Cu") (at 192.01775 86.326748 180)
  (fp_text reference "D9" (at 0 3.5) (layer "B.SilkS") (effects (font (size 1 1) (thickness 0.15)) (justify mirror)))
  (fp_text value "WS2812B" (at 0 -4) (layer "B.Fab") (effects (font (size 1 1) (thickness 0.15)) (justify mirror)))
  (pad "1" smd rect (at -2.45 1.65 180) (size 1.5 0.9) (layers "B.Cu" "B.Paste" "B.Mask") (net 22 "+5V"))
  (pad "2" smd rect (at -2.45 -1.65 180) (size 1.5 0.9) (layers "B.Cu" "B.Paste" "B.Mask") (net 24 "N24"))
  (pad "3" smd rect (at 2.45 -1.65 180) (size 1.5 0.9) (layers "B.Cu" "B.Paste" "B.Mask") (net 2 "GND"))
  (pad "4" smd rect (at 2.45 1.65 180) (size 1.5 0.9) (layers "B.Cu" "B.Paste" "B.Mask") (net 49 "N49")))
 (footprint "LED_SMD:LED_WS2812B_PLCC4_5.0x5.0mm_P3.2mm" (layer "B.Cu") (at 111.05525 118.870498 180)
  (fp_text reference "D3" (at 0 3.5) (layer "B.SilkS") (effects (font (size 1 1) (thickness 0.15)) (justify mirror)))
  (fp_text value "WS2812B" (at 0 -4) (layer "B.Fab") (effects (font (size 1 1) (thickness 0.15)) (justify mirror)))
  (pad "1" smd rect (at -2.45 1.65 180) (size 1.5 0.9) (layers "B.Cu" "B.Paste" "B.Mask") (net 22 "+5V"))
  (pad "2" smd rect (at -2.45 -1.65 180) (size 1.5 0.9) (layers "B.Cu" "B.Paste" "B.Mask") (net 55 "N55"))
  (pad "3" smd rect (at 2.45 -1.65 180) (size 1.5 0.9) (layers "B.Cu" "B.Paste" "B.Mask") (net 2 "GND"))
  (pad "4" smd rect (at 2.45 1.65 180) (size 1.5 0.9) (layers "B.Cu" "B.Paste" "B.Mask") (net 53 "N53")))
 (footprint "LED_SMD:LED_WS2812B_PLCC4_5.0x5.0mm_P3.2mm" (layer "B.Cu") (at 153.91775 124.426748 180)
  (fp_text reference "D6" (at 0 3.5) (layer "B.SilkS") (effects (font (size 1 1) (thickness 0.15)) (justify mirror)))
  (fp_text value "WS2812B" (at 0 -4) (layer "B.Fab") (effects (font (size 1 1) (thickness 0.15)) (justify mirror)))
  (pad "1" smd rect (at -2.45 1.65 180) (size 1.5 0.9) (layers "B.Cu" "B.Paste" "B.Mask") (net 22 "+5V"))
  (pad "2" smd rect (at -2.45 -1.65 180) (size 1.5 0.9) (layers "B.Cu" "B.Paste" "B.Mask") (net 52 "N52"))
  (pad "3" smd rect (at 2.45 -1.65 180) (size 1.5 0.9) (layers "B.Cu" "B.Paste" "B.Mask") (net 2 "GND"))
  (pad "4" smd rect (at 2.45 1.65 180) (size 1.5 0.9) (layers "B.Cu" "B.Paste" "B.Mask") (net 48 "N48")))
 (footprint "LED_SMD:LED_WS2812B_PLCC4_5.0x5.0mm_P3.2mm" (layer "B.Cu") (at 92.00525 86.326748 180)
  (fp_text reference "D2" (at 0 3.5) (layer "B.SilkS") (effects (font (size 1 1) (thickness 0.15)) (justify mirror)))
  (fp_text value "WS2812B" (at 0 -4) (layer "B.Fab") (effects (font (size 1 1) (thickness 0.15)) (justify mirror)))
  (pad "1" smd rect (at -2.45 1.65 180) (size 1.5 0.9) (layers "B.Cu" "B.Paste" "B.Mask") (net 22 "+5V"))
  (pad "2" smd rect (at -2.45 -1.65 180) (size 1.5 0.9) (layers "B.Cu" "B.Paste" "B.Mask") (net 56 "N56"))
  (pad "3" smd rect (at 2.45 -1.65 180) (size 1.5 0.9) (layers "B.Cu" "B.Paste" "B.Mask") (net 2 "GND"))
  (pad "4" smd rect (at 2.45 1.65 180) (size 1.5 0.9) (layers "B.Cu" "B.Paste" "B.Mask") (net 51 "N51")))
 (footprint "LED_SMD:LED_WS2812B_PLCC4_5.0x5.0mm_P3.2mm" (layer "B.Cu") (at 130.10525 124.426748 180)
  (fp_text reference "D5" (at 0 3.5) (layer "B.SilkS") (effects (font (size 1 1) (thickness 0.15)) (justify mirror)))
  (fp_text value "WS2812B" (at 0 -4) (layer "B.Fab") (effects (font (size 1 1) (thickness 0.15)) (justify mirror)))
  (pad "1" smd rect (at -2.45 1.65 180) (size 1.5 0.9) (layers "B.Cu" "B.Paste" "B.Mask") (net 22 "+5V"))
  (pad "2" smd rect (at -2.45 -1.65 180) (size 1.5 0.9) (layers "B.Cu" "B.Paste" "B.Mask") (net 50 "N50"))
  (pad "3" smd rect (at 2.45 -1.65 180) (size 1.5 0.9) (layers "B.Cu" "B.Paste" "B.Mask") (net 2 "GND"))
  (pad "4" smd rect (at 2.45 1.65 180) (size 1.5 0.9) (layers "B.Cu" "B.Paste" "B.Mask") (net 55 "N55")))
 (gr_line (start 84.1375 59.53125) (end 200.025 59.53125) (layer "Edge.Cuts") (width 0.1))
 (gr_line (start 81.75625 127.79375) (end 81.75625 61.9125) (layer "Edge.Cuts") (width 0.1))
 (gr_arc (start 81.75625 61.9125) (mid 82.453702 60.228702) (end 84.1375 59.53125) (layer "Edge.Cuts") (width 0.1))
 (gr_arc (start 200.025 59.53125) (mid 201.708798 60.228702) (end 202.40625 61.9125) (layer "Edge.Cuts") (width 0.1))
 (gr_line (start 200.025 130.175) (end 84.1375 130.175) (layer "Edge.Cuts") (width 0.1))
 (gr_arc (start 84.1375 130.175) (mid 82.453702 129.477548) (end 81.75625 127.79375) (layer "Edge.Cuts") (width 0.1))
 (gr_line (start 202.40625 61.9125) (end 202.40625 127.79375) (layer "Edge.Cuts") (width 0.1))
 (gr_arc (start 202.40625 127.79375) (mid 201.708798 129.477548) (end 200.025 130.175) (layer "Edge.Cuts") (width 0.1))
 (segment (start 153.19375 79.375) (end 157.1625 79.375) (width 0.254) (layer "F.Cu") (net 8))
 (segment (start 150.1775 73.66) (end 150.8125 74.295) (width 0.254) (layer "F.Cu") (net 8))
 (segment (start 161.891748 81.722998) (end 164.07775 81.722998) (width 0.254) (layer "F.Cu") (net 8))
 (segment (start 161.891748 81.722998) (end 159.510498 81.722998) (width 0.254) (layer "F.Cu") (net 8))
 (segment (start 159.510498 81.722998) (end 157.1625 79.375) (width 0.254) (layer "F.Cu") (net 8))
 (segment (start 150.8125 74.295) (end 150.8125 76.99375) (width 0.254) (layer "F.Cu") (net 8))
 (segment (start 150.8125 76.99375) (end 153.19375 79.375) (width 0.254) (layer "F.Cu") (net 8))
 (segment (start 152.7175 82.07375) (end 154.906748 84.262998) (width 0.381) (layer "F.Cu") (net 9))
 (segment (start 152.7175 81.28) (end 152.7175 82.07375) (width 0.381) (layer "F.Cu") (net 9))
 (segment (start 154.906748 84.262998) (end 164.07775 84.262998) (width 0.381) (layer "F.Cu") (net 9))
 (segment (start 150.1775 111.76) (end 157.32125 111.76) (width 0.254) (layer "F.Cu") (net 16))
 (segment (start 161.958252 107.122998) (end 164.07775 107.122998) (width 0.254) (layer "F.Cu") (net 16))
 (segment (start 157.32125 111.76) (end 161.958252 107.122998) (width 0.254) (layer "F.Cu") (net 16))
 (segment (start 161.13125 117.475) (end 164.07775 114.5285) (width 0.381) (layer "F.Cu") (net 17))
 (segment (start 154.6225 117.475) (end 161.13125 117.475) (width 0.381) (layer "F.Cu") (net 17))
 (segment (start 152.7175 119.38) (end 154.6225 117.475) (width 0.381) (layer "F.Cu") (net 17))
 (segment (start 164.07775 114.5285) (end 164.07775 109.662998) (width 0.381) (layer "F.Cu") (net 17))
 (segment (start 174.625 97.63125) (end 176.2125 96.04375) (width 0.381) (layer "F.Cu") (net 11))
 (segment (start 171.69775 100.137998) (end 171.69775 98.760748) (width 0.381) (layer "F.Cu") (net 11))
 (segment (start 173.0375 86.51875) (end 179.3875 80.16875) (width 0.381) (layer "F.Cu") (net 11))
 (segment (start 179.3875 74.033248) (end 181.85775 71.562998) (width 0.381) (layer "F.Cu") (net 11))
 (segment (start 173.0375 90.4875) (end 173.0375 86.51875) (width 0.381) (layer "F.Cu") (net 11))
 (segment (start 172.827249 97.63125) (end 174.625 97.63125) (width 0.381) (layer "F.Cu") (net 11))
 (segment (start 176.2125 96.04375) (end 176.2125 93.6625) (width 0.381) (layer "F.Cu") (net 11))
 (segment (start 176.2125 93.6625) (end 173.0375 90.4875) (width 0.381) (layer "F.Cu") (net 11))
 (segment (start 171.69775 98.760748) (end 172.827249 97.63125) (width 0.381) (layer "F.Cu") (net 11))
 (segment (start 179.3875 80.16875) (end 179.3875 74.033248) (width 0.381) (layer "F.Cu") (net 11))
 (segment (start 183.145999 61.402998) (end 181.85775 61.402998) (width 0.254) (layer "F.Cu") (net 20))
 (segment (start 188.20775 73.467998) (end 188.20775 66.464749) (width 0.254) (layer "F.Cu") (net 20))
 (segment (start 188.20775 66.464749) (end 183.145999 61.402998) (width 0.254) (layer "F.Cu") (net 20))
 (segment (start 181.85775 61.402998) (end 183.47175 61.402998) (width 0.254) (layer "B.Cu") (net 20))
 (segment (start 190.74775 81.087998) (end 189.831748 81.087998) (width 0.254) (layer "F.Cu") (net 21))
 (segment (start 185.685749 76.941999) (end 185.685749 65.829499) (width 0.381) (layer "F.Cu") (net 21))
 (segment (start 189.831748 81.087998) (end 185.685749 76.941999) (width 0.381) (layer "F.Cu") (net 21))
 (segment (start 183.799248 63.942998) (end 181.85775 63.942998) (width 0.381) (layer "F.Cu") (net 21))
 (segment (start 185.685749 65.829499) (end 183.799248 63.942998) (width 0.381) (layer "F.Cu") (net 21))
 (segment (start 184.94375 77.7875) (end 184.94375 75.40625) (width 0.254) (layer "F.Cu") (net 1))
 (segment (start 184.94375 75.40625) (end 183.640498 74.102998) (width 0.254) (layer "F.Cu") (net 1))
 (segment (start 188.11875 111.478998) (end 188.11875 80.9625) (width 0.254) (layer "F.Cu") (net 1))
 (segment (start 183.640498 74.102998) (end 181.85775 74.102998) (width 0.254) (layer "F.Cu") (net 1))
 (segment (start 188.11875 80.9625) (end 184.94375 77.7875) (width 0.254) (layer "F.Cu") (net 1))
 (segment (start 188.20775 111.567998) (end 188.11875 111.478998) (width 0.254) (layer "F.Cu") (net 1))
 (segment (start 182.608623 76.642998) (end 181.85775 76.642998) (width 0.381) (layer "F.Cu") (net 3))
 (segment (start 186.53125 116.68125) (end 184.94375 115.09375) (width 0.381) (layer "F.Cu") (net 3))
 (segment (start 184.94375 78.978125) (end 182.608623 76.642998) (width 0.381) (layer "F.Cu") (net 3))
 (segment (start 187.650602 116.68125) (end 186.53125 116.68125) (width 0.381) (layer "F.Cu") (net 3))
 (segment (start 190.74775 119.187998) (end 190.15735 119.187998) (width 0.381) (layer "F.Cu") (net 3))
 (segment (start 190.15735 119.187998) (end 187.650602 116.68125) (width 0.381) (layer "F.Cu") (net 3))
 (segment (start 184.94375 115.09375) (end 184.94375 78.978125) (width 0.381) (layer "F.Cu") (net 3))
 (segment (start 178.59375 72.286998) (end 181.85775 69.022998) (width 0.254) (layer "F.Cu") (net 10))
 (segment (start 169.15775 88.811) (end 178.59375 79.375) (width 0.254) (layer "F.Cu") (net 10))
 (segment (start 178.59375 79.375) (end 178.59375 72.286998) (width 0.254) (layer "F.Cu") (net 10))
 (segment (start 169.15775 92.517998) (end 169.15775 88.811) (width 0.254) (layer "F.Cu") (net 10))
 (segment (start 180.941748 94.422998) (end 181.85775 94.422998) (width 0.254) (layer "F.Cu") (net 29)))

